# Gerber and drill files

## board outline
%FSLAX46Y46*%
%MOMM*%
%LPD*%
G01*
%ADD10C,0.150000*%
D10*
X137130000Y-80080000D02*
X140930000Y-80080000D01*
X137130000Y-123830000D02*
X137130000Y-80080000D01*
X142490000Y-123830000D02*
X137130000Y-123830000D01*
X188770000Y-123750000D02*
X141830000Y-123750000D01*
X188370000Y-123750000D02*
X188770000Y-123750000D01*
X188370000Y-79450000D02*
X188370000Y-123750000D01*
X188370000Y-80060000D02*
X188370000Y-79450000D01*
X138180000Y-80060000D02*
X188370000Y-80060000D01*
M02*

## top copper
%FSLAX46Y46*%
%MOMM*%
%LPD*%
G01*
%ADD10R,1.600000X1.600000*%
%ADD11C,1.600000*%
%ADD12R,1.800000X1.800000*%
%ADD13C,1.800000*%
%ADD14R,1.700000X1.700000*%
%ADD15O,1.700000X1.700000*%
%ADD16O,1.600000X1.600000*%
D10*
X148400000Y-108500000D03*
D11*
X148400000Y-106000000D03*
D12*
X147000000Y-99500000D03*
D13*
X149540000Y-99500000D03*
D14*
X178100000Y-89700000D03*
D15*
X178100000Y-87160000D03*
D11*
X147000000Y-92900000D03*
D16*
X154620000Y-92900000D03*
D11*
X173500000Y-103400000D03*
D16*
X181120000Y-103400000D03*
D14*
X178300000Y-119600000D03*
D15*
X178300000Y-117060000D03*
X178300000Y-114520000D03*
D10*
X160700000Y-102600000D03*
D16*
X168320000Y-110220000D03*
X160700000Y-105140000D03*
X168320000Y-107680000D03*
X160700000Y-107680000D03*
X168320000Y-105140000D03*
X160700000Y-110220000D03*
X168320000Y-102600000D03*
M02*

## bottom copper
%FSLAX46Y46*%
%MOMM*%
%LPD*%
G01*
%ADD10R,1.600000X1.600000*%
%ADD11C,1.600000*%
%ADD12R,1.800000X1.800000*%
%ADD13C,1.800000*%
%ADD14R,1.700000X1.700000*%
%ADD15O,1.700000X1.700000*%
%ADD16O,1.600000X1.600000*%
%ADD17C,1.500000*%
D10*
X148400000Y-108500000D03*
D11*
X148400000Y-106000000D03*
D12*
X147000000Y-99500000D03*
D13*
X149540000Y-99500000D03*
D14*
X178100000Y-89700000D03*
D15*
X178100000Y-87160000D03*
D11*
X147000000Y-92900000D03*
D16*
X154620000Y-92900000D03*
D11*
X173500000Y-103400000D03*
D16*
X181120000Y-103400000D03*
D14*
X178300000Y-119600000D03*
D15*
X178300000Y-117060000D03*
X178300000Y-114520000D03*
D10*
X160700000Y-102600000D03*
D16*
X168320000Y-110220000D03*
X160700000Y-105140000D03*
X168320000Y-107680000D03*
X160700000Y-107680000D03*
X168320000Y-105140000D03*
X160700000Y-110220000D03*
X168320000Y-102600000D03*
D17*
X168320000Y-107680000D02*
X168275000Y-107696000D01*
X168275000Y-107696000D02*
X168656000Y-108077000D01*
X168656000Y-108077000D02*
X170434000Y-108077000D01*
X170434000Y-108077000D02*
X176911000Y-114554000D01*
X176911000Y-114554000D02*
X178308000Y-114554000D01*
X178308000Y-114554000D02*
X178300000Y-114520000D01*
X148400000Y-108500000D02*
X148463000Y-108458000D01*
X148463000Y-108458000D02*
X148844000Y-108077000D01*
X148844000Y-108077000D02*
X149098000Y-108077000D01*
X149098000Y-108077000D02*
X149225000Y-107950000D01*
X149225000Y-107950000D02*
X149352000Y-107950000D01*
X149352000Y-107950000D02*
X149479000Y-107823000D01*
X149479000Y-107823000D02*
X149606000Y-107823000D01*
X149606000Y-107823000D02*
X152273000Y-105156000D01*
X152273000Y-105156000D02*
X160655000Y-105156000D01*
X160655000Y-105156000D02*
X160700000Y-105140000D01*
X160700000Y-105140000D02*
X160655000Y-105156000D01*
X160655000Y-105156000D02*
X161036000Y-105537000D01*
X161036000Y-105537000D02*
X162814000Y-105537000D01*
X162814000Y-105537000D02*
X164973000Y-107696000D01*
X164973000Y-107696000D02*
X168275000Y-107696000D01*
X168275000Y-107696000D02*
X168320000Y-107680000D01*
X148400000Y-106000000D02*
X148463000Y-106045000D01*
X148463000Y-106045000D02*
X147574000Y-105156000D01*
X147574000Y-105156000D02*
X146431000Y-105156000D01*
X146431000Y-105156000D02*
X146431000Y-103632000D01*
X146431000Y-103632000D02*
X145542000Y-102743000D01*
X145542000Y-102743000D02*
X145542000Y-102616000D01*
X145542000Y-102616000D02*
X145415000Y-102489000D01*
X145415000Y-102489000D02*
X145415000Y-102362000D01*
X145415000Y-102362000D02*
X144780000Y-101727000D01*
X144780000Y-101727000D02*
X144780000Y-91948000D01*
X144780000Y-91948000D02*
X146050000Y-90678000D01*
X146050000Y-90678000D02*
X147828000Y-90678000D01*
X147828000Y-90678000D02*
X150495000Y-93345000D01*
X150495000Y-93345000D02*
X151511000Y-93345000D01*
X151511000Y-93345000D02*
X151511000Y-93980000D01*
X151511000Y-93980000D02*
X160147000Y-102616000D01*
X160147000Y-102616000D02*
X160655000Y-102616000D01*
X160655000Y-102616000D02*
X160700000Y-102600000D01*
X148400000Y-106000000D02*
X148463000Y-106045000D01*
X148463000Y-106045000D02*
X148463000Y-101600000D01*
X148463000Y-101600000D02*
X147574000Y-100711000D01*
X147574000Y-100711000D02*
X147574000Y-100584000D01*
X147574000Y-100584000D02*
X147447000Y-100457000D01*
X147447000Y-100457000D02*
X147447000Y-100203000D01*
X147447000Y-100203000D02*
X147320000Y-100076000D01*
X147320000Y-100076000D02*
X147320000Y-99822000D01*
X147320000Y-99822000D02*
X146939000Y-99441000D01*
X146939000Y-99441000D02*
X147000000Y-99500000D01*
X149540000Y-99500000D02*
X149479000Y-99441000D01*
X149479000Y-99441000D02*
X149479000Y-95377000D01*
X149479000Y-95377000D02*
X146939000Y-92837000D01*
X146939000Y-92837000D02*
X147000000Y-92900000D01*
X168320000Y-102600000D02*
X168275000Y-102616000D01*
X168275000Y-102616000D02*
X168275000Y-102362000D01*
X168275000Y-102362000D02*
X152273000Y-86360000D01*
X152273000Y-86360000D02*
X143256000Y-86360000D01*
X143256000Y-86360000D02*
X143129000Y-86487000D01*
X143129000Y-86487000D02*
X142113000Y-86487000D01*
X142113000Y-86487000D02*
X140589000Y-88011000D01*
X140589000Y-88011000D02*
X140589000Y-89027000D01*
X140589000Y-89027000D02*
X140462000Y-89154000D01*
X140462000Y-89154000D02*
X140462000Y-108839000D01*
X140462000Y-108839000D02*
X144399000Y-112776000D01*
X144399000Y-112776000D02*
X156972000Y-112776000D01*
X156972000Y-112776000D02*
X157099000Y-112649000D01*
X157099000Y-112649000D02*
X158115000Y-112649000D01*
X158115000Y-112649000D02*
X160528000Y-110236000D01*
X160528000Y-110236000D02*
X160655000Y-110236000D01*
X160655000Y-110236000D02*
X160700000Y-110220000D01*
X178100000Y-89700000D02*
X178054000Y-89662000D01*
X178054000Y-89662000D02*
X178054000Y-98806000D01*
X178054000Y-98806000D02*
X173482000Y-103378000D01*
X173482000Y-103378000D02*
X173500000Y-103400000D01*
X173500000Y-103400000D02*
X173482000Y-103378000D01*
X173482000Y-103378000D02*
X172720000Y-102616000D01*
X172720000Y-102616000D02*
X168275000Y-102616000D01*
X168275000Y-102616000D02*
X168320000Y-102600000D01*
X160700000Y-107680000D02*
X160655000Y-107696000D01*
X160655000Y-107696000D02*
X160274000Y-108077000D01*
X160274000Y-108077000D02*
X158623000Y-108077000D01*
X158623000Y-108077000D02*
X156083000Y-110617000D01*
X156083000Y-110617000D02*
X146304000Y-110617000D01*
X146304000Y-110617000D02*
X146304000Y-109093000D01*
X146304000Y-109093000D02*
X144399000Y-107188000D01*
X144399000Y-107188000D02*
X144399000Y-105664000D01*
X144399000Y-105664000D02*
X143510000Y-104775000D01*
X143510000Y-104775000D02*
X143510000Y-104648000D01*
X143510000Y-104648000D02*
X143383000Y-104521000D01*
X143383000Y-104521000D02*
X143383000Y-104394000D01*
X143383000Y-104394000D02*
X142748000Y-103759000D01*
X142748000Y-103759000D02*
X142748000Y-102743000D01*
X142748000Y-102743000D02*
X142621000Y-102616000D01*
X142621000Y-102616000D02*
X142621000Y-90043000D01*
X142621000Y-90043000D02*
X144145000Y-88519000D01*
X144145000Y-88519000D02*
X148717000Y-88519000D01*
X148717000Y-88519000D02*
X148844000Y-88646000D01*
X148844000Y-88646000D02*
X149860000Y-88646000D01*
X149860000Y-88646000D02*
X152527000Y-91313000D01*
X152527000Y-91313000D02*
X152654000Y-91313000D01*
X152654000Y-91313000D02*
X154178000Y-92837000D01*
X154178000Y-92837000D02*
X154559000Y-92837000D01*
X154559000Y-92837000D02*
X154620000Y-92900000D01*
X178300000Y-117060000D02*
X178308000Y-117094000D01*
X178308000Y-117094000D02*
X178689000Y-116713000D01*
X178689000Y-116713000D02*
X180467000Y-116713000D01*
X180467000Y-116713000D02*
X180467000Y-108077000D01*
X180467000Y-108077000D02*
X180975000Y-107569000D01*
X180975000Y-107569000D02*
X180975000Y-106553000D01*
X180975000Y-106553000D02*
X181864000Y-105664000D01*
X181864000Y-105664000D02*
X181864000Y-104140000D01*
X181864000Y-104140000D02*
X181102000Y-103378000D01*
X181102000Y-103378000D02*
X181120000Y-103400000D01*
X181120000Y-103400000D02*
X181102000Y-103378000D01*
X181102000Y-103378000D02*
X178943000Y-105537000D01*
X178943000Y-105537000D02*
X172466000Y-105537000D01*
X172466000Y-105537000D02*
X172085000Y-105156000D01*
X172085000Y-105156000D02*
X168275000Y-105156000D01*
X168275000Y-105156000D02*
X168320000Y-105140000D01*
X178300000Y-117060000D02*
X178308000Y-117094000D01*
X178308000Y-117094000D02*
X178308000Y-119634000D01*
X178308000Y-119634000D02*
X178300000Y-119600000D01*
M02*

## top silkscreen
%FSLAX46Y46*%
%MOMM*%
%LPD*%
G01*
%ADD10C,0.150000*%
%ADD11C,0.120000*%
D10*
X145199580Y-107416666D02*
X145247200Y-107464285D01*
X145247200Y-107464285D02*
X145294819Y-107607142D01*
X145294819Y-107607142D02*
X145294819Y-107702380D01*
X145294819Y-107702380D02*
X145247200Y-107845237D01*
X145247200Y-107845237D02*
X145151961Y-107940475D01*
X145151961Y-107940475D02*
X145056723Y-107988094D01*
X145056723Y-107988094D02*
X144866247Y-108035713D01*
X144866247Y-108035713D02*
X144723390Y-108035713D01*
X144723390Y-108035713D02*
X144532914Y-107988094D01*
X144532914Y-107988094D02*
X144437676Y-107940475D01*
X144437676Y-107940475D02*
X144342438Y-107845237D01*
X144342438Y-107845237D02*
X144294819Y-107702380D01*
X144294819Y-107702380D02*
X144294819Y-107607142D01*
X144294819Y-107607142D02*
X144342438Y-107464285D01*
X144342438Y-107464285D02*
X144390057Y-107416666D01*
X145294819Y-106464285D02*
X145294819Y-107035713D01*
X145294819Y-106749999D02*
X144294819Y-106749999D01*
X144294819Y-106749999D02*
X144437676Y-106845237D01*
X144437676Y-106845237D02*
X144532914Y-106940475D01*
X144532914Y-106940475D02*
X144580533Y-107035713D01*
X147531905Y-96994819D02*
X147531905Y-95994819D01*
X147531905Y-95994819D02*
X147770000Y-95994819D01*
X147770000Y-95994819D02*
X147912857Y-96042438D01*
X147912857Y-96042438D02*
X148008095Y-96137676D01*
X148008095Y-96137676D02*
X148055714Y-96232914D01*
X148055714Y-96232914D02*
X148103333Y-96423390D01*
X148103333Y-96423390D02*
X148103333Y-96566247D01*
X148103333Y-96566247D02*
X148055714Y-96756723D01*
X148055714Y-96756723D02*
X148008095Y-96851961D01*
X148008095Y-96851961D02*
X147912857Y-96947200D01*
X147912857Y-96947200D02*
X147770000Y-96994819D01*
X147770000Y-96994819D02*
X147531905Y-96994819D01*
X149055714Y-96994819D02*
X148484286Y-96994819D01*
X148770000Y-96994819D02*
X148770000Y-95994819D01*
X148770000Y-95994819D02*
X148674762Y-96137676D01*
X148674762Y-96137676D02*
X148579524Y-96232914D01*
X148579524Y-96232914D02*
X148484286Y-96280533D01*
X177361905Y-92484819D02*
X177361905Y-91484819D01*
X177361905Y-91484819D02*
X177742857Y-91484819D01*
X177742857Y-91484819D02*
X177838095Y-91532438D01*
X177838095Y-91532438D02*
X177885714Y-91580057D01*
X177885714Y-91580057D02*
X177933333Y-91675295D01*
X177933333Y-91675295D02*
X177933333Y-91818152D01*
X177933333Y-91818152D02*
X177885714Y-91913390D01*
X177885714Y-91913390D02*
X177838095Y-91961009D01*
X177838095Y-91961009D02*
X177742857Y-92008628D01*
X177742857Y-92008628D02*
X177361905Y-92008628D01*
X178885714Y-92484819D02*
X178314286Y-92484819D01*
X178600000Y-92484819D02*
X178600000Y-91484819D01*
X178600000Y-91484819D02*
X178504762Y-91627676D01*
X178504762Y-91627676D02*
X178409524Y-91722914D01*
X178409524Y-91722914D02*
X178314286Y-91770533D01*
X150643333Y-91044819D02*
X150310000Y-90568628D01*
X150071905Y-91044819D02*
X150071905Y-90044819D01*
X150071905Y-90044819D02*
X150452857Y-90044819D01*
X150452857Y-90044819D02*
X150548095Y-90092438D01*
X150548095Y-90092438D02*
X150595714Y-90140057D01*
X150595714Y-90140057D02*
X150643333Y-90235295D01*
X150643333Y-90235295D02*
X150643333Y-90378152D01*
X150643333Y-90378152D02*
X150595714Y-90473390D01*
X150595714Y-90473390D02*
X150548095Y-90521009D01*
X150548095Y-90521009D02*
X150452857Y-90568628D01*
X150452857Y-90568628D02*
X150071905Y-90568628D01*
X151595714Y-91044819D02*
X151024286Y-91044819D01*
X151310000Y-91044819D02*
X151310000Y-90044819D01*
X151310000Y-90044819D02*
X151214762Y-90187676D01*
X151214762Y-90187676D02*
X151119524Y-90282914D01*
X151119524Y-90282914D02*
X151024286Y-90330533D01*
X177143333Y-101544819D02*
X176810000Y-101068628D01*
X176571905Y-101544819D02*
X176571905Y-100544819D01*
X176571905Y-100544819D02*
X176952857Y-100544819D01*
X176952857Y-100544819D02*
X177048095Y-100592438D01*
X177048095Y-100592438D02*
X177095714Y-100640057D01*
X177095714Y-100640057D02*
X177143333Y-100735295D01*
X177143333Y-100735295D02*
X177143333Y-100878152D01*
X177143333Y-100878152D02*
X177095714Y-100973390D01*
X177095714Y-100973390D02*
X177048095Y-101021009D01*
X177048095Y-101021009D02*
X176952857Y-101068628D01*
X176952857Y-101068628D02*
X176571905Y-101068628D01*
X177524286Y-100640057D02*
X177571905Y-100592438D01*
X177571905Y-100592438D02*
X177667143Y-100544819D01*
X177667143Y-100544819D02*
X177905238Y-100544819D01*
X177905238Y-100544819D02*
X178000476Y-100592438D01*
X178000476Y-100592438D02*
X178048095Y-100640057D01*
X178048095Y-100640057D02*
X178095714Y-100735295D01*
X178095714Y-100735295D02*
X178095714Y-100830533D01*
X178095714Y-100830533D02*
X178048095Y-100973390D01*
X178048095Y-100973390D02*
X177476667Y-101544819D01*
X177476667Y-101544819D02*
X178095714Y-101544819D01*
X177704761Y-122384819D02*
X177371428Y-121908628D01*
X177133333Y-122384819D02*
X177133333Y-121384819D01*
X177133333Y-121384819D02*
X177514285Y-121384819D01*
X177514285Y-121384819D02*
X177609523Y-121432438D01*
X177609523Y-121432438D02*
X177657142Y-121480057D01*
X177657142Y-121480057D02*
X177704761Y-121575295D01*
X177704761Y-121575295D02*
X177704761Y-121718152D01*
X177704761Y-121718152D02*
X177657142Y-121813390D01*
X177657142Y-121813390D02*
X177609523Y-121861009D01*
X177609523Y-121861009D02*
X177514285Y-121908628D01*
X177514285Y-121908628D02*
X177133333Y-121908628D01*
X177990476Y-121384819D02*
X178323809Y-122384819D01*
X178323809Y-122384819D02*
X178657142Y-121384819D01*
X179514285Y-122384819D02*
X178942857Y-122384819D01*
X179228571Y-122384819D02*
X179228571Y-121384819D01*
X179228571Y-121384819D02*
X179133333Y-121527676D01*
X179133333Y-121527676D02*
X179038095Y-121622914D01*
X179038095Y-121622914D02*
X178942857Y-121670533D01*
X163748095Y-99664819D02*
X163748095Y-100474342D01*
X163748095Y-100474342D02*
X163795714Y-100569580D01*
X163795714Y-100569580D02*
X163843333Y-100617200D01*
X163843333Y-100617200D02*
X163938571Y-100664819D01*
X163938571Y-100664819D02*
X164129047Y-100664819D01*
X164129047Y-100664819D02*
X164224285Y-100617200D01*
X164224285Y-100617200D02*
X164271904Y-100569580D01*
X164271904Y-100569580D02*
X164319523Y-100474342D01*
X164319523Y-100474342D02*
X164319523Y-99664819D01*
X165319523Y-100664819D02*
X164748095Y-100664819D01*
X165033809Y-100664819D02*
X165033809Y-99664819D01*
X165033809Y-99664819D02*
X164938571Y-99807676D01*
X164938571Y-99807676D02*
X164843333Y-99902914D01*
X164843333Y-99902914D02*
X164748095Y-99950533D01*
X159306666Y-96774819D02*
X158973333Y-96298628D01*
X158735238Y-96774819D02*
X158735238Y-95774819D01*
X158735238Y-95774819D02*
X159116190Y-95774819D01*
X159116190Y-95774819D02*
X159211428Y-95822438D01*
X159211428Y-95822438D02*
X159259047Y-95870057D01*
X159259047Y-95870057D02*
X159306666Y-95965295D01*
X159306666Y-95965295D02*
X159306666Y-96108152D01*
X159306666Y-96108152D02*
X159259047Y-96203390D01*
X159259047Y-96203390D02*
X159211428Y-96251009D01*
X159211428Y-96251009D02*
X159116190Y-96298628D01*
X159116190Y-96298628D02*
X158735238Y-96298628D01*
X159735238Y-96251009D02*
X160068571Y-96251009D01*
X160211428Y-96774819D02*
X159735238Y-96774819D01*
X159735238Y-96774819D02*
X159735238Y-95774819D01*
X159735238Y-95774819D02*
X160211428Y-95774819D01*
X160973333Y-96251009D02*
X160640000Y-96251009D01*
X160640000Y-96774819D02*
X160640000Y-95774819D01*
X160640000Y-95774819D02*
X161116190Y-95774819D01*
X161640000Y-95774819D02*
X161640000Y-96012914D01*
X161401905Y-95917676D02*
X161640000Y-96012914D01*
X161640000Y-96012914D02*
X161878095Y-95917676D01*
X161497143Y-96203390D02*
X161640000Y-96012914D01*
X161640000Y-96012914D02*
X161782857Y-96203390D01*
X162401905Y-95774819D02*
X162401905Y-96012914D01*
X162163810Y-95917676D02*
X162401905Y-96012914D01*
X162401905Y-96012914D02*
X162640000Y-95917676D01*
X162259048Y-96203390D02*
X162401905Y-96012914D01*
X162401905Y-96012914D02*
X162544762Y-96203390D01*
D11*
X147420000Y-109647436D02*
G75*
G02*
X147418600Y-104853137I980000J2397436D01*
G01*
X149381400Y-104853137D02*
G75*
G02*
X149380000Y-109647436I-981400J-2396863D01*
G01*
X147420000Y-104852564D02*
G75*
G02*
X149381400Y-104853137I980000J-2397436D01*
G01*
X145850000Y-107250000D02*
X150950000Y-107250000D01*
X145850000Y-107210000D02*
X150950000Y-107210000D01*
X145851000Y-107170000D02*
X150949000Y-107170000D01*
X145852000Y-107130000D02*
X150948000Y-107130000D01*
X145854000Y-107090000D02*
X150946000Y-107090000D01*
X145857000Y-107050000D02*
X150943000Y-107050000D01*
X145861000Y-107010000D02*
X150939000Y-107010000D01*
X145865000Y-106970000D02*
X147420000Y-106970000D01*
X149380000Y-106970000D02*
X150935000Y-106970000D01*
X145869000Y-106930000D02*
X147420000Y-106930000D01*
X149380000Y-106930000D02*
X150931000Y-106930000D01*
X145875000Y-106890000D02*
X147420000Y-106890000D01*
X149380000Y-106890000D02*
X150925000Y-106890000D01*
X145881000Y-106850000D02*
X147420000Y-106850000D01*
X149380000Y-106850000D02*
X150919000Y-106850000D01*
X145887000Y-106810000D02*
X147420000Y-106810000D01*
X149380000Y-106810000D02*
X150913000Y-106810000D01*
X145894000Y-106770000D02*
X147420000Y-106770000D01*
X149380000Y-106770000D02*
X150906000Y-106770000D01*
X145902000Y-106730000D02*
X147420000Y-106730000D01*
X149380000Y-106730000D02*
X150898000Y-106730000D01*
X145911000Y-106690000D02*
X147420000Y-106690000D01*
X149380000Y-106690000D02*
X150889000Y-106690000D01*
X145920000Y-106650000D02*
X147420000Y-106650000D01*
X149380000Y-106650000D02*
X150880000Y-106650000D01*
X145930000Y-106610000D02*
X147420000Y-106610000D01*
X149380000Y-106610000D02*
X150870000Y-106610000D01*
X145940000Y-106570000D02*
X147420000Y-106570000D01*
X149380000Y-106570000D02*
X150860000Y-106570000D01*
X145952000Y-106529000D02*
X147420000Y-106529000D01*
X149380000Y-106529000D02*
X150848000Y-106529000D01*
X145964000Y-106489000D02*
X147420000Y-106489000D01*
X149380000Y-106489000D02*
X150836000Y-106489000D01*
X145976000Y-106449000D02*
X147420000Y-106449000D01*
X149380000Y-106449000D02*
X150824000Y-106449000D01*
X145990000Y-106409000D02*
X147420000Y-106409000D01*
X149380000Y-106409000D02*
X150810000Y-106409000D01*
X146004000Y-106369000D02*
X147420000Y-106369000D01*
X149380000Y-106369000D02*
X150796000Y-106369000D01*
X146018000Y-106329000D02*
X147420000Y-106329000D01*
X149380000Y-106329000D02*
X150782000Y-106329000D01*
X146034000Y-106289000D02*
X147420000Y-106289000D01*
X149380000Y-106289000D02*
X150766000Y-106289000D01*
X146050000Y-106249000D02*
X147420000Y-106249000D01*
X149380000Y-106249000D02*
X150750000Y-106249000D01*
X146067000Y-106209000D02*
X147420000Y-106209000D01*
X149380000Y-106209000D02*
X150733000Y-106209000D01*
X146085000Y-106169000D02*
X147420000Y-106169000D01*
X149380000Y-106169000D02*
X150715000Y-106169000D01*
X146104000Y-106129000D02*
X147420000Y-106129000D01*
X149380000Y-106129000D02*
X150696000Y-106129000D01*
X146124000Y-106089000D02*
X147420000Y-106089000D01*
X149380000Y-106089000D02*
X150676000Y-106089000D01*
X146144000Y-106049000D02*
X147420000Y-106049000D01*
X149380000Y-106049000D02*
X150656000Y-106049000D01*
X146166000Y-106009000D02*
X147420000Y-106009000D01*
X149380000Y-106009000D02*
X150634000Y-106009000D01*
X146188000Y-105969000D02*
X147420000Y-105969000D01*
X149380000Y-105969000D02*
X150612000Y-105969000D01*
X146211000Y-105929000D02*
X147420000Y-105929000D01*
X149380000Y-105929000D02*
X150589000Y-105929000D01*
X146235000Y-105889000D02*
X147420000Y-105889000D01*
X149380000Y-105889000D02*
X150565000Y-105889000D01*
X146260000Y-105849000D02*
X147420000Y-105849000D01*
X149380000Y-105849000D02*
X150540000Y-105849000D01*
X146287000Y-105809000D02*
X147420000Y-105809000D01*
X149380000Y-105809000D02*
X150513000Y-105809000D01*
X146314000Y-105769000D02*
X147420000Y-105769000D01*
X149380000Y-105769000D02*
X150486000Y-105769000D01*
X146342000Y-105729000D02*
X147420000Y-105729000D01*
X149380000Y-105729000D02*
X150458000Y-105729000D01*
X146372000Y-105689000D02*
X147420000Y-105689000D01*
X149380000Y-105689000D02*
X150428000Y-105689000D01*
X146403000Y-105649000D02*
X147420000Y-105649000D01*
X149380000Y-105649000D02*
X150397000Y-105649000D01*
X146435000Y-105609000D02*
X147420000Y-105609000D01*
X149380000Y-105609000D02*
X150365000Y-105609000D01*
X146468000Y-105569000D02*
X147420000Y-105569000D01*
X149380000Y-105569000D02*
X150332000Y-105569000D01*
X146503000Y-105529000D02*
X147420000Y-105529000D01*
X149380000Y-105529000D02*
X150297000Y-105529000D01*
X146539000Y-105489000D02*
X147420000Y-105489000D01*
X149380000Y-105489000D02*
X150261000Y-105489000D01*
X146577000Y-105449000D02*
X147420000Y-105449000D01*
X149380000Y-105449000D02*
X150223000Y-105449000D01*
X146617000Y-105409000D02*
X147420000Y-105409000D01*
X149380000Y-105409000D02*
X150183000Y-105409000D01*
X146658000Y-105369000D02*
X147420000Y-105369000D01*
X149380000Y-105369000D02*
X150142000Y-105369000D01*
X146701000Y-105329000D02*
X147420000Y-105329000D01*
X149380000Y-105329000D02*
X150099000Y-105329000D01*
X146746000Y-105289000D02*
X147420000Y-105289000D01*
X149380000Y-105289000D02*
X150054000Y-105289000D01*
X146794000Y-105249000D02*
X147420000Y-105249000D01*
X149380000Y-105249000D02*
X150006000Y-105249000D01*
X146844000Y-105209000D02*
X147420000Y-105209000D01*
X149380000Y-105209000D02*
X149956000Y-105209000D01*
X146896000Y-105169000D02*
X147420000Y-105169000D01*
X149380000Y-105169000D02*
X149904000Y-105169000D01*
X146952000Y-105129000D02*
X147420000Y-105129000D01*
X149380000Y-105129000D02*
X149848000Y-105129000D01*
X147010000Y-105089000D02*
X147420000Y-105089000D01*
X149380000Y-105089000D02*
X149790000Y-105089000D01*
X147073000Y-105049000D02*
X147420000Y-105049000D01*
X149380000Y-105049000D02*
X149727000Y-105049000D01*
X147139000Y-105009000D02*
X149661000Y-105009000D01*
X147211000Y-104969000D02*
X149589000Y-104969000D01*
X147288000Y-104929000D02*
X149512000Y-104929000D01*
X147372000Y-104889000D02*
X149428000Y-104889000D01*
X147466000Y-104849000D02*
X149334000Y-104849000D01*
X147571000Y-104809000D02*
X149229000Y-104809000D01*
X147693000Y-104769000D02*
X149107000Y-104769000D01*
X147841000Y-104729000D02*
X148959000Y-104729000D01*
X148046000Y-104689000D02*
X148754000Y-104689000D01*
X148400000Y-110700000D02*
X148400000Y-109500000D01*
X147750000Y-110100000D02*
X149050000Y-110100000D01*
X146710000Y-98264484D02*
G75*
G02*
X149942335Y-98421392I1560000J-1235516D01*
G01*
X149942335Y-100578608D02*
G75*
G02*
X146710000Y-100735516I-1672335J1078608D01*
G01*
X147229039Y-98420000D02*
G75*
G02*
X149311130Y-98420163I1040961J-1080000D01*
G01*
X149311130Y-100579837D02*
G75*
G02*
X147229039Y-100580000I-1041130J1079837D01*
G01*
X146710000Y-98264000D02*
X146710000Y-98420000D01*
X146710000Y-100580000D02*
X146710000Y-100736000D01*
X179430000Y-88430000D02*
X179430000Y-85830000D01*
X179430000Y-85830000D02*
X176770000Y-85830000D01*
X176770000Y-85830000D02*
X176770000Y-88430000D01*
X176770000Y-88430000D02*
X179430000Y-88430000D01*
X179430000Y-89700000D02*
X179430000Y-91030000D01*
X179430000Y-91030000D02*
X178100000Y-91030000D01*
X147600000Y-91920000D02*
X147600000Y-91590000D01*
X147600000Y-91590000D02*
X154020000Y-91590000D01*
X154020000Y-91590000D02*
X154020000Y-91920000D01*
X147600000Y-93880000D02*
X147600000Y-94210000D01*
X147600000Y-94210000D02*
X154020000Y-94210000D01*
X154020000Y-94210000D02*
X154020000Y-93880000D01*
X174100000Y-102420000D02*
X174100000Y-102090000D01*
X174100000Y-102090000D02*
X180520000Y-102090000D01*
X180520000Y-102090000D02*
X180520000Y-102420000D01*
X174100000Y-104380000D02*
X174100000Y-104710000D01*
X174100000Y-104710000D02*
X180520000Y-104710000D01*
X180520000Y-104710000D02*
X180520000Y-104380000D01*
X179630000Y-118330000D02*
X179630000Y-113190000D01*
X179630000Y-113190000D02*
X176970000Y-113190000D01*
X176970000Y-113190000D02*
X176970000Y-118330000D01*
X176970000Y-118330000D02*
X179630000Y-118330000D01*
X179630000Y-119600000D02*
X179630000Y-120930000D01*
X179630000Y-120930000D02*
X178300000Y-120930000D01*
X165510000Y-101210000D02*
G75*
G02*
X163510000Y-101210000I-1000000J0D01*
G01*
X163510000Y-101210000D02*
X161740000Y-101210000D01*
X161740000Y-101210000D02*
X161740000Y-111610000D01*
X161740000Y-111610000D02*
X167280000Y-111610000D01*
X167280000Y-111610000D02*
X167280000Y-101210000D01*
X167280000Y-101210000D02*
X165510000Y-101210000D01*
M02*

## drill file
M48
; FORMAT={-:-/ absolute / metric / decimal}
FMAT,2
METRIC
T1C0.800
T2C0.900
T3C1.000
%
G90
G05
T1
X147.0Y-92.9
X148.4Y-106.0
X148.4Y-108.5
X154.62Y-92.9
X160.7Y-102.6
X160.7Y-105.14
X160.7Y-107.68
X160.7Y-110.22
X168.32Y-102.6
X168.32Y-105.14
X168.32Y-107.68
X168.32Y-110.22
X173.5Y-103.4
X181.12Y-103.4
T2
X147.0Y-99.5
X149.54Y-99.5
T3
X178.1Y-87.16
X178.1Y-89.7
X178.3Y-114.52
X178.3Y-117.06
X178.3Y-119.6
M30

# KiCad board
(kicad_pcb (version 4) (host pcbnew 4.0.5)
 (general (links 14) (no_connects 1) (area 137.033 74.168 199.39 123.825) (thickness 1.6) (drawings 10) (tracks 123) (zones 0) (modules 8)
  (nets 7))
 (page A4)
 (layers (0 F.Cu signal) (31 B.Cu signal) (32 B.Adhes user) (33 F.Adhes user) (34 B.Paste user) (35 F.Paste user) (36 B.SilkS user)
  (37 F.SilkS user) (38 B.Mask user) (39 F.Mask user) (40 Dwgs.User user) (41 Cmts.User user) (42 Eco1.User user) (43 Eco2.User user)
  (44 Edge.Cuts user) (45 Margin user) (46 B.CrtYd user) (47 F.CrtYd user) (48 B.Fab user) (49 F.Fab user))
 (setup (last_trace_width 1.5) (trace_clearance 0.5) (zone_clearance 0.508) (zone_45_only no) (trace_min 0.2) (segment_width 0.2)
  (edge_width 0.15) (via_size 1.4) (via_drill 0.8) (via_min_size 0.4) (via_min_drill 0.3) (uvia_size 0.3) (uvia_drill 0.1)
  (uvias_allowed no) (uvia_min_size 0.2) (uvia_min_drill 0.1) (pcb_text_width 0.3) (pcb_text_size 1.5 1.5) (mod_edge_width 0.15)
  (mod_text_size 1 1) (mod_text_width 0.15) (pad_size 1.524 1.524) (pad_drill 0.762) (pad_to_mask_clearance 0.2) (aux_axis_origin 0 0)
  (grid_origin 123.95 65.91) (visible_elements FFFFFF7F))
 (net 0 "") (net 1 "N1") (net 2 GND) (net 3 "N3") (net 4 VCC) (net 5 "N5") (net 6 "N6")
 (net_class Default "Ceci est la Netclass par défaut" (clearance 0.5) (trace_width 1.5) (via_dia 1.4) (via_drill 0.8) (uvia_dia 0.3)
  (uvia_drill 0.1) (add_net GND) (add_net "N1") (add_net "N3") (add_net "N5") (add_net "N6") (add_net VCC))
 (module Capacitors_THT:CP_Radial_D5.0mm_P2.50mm (layer F.Cu) (at 148.4 108.5 90)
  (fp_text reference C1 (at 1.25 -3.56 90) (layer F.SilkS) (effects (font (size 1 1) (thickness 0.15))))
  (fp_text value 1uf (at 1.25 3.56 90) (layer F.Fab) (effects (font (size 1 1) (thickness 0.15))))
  (fp_arc (start 1.25 0) (end -1.147436 -0.98) (angle 135.5) (layer F.SilkS) (width 0.12))
  (fp_arc (start 1.25 0) (end -1.147436 0.98) (angle -135.5) (layer F.SilkS) (width 0.12))
  (fp_arc (start 1.25 0) (end 3.647436 -0.98) (angle 44.5) (layer F.SilkS) (width 0.12))
  (fp_line (start 1.25 -2.55) (end 1.25 2.55) (layer F.SilkS) (width 0.12))
  (fp_line (start 1.29 -2.55) (end 1.29 2.55) (layer F.SilkS) (width 0.12))
  (fp_line (start 1.33 -2.549) (end 1.33 2.549) (layer F.SilkS) (width 0.12))
  (fp_line (start 1.37 -2.548) (end 1.37 2.548) (layer F.SilkS) (width 0.12))
  (fp_line (start 1.41 -2.546) (end 1.41 2.546) (layer F.SilkS) (width 0.12))
  (fp_line (start 1.45 -2.543) (end 1.45 2.543) (layer F.SilkS) (width 0.12))
  (fp_line (start 1.49 -2.539) (end 1.49 2.539) (layer F.SilkS) (width 0.12))
  (fp_line (start 1.53 -2.535) (end 1.53 -0.98) (layer F.SilkS) (width 0.12))
  (fp_line (start 1.53 0.98) (end 1.53 2.535) (layer F.SilkS) (width 0.12))
  (fp_line (start 1.57 -2.531) (end 1.57 -0.98) (layer F.SilkS) (width 0.12))
  (fp_line (start 1.57 0.98) (end 1.57 2.531) (layer F.SilkS) (width 0.12))
  (fp_line (start 1.61 -2.525) (end 1.61 -0.98) (layer F.SilkS) (width 0.12))
  (fp_line (start 1.61 0.98) (end 1.61 2.525) (layer F.SilkS) (width 0.12))
  (fp_line (start 1.65 -2.519) (end 1.65 -0.98) (layer F.SilkS) (width 0.12))
  (fp_line (start 1.65 0.98) (end 1.65 2.519) (layer F.SilkS) (width 0.12))
  (fp_line (start 1.69 -2.513) (end 1.69 -0.98) (layer F.SilkS) (width 0.12))
  (fp_line (start 1.69 0.98) (end 1.69 2.513) (layer F.SilkS) (width 0.12))
  (fp_line (start 1.73 -2.506) (end 1.73 -0.98) (layer F.SilkS) (width 0.12))
  (fp_line (start 1.73 0.98) (end 1.73 2.506) (layer F.SilkS) (width 0.12))
  (fp_line (start 1.77 -2.498) (end 1.77 -0.98) (layer F.SilkS) (width 0.12))
  (fp_line (start 1.77 0.98) (end 1.77 2.498) (layer F.SilkS) (width 0.12))
  (fp_line (start 1.81 -2.489) (end 1.81 -0.98) (layer F.SilkS) (width 0.12))
  (fp_line (start 1.81 0.98) (end 1.81 2.489) (layer F.SilkS) (width 0.12))
  (fp_line (start 1.85 -2.48) (end 1.85 -0.98) (layer F.SilkS) (width 0.12))
  (fp_line (start 1.85 0.98) (end 1.85 2.48) (layer F.SilkS) (width 0.12))
  (fp_line (start 1.89 -2.47) (end 1.89 -0.98) (layer F.SilkS) (width 0.12))
  (fp_line (start 1.89 0.98) (end 1.89 2.47) (layer F.SilkS) (width 0.12))
  (fp_line (start 1.93 -2.46) (end 1.93 -0.98) (layer F.SilkS) (width 0.12))
  (fp_line (start 1.93 0.98) (end 1.93 2.46) (layer F.SilkS) (width 0.12))
  (fp_line (start 1.971 -2.448) (end 1.971 -0.98) (layer F.SilkS) (width 0.12))
  (fp_line (start 1.971 0.98) (end 1.971 2.448) (layer F.SilkS) (width 0.12))
  (fp_line (start 2.011 -2.436) (end 2.011 -0.98) (layer F.SilkS) (width 0.12))
  (fp_line (start 2.011 0.98) (end 2.011 2.436) (layer F.SilkS) (width 0.12))
  (fp_line (start 2.051 -2.424) (end 2.051 -0.98) (layer F.SilkS) (width 0.12))
  (fp_line (start 2.051 0.98) (end 2.051 2.424) (layer F.SilkS) (width 0.12))
  (fp_line (start 2.091 -2.41) (end 2.091 -0.98) (layer F.SilkS) (width 0.12))
  (fp_line (start 2.091 0.98) (end 2.091 2.41) (layer F.SilkS) (width 0.12))
  (fp_line (start 2.131 -2.396) (end 2.131 -0.98) (layer F.SilkS) (width 0.12))
  (fp_line (start 2.131 0.98) (end 2.131 2.396) (layer F.SilkS) (width 0.12))
  (fp_line (start 2.171 -2.382) (end 2.171 -0.98) (layer F.SilkS) (width 0.12))
  (fp_line (start 2.171 0.98) (end 2.171 2.382) (layer F.SilkS) (width 0.12))
  (fp_line (start 2.211 -2.366) (end 2.211 -0.98) (layer F.SilkS) (width 0.12))
  (fp_line (start 2.211 0.98) (end 2.211 2.366) (layer F.SilkS) (width 0.12))
  (fp_line (start 2.251 -2.35) (end 2.251 -0.98) (layer F.SilkS) (width 0.12))
  (fp_line (start 2.251 0.98) (end 2.251 2.35) (layer F.SilkS) (width 0.12))
  (fp_line (start 2.291 -2.333) (end 2.291 -0.98) (layer F.SilkS) (width 0.12))
  (fp_line (start 2.291 0.98) (end 2.291 2.333) (layer F.SilkS) (width 0.12))
  (fp_line (start 2.331 -2.315) (end 2.331 -0.98) (layer F.SilkS) (width 0.12))
  (fp_line (start 2.331 0.98) (end 2.331 2.315) (layer F.SilkS) (width 0.12))
  (fp_line (start 2.371 -2.296) (end 2.371 -0.98) (layer F.SilkS) (width 0.12))
  (fp_line (start 2.371 0.98) (end 2.371 2.296) (layer F.SilkS) (width 0.12))
  (fp_line (start 2.411 -2.276) (end 2.411 -0.98) (layer F.SilkS) (width 0.12))
  (fp_line (start 2.411 0.98) (end 2.411 2.276) (layer F.SilkS) (width 0.12))
  (fp_line (start 2.451 -2.256) (end 2.451 -0.98) (layer F.SilkS) (width 0.12))
  (fp_line (start 2.451 0.98) (end 2.451 2.256) (layer F.SilkS) (width 0.12))
  (fp_line (start 2.491 -2.234) (end 2.491 -0.98) (layer F.SilkS) (width 0.12))
  (fp_line (start 2.491 0.98) (end 2.491 2.234) (layer F.SilkS) (width 0.12))
  (fp_line (start 2.531 -2.212) (end 2.531 -0.98) (layer F.SilkS) (width 0.12))
  (fp_line (start 2.531 0.98) (end 2.531 2.212) (layer F.SilkS) (width 0.12))
  (fp_line (start 2.571 -2.189) (end 2.571 -0.98) (layer F.SilkS) (width 0.12))
  (fp_line (start 2.571 0.98) (end 2.571 2.189) (layer F.SilkS) (width 0.12))
  (fp_line (start 2.611 -2.165) (end 2.611 -0.98) (layer F.SilkS) (width 0.12))
  (fp_line (start 2.611 0.98) (end 2.611 2.165) (layer F.SilkS) (width 0.12))
  (fp_line (start 2.651 -2.14) (end 2.651 -0.98) (layer F.SilkS) (width 0.12))
  (fp_line (start 2.651 0.98) (end 2.651 2.14) (layer F.SilkS) (width 0.12))
  (fp_line (start 2.691 -2.113) (end 2.691 -0.98) (layer F.SilkS) (width 0.12))
  (fp_line (start 2.691 0.98) (end 2.691 2.113) (layer F.SilkS) (width 0.12))
  (fp_line (start 2.731 -2.086) (end 2.731 -0.98) (layer F.SilkS) (width 0.12))
  (fp_line (start 2.731 0.98) (end 2.731 2.086) (layer F.SilkS) (width 0.12))
  (fp_line (start 2.771 -2.058) (end 2.771 -0.98) (layer F.SilkS) (width 0.12))
  (fp_line (start 2.771 0.98) (end 2.771 2.058) (layer F.SilkS) (width 0.12))
  (fp_line (start 2.811 -2.028) (end 2.811 -0.98) (layer F.SilkS) (width 0.12))
  (fp_line (start 2.811 0.98) (end 2.811 2.028) (layer F.SilkS) (width 0.12))
  (fp_line (start 2.851 -1.997) (end 2.851 -0.98) (layer F.SilkS) (width 0.12))
  (fp_line (start 2.851 0.98) (end 2.851 1.997) (layer F.SilkS) (width 0.12))
  (fp_line (start 2.891 -1.965) (end 2.891 -0.98) (layer F.SilkS) (width 0.12))
  (fp_line (start 2.891 0.98) (end 2.891 1.965) (layer F.SilkS) (width 0.12))
  (fp_line (start 2.931 -1.932) (end 2.931 -0.98) (layer F.SilkS) (width 0.12))
  (fp_line (start 2.931 0.98) (end 2.931 1.932) (layer F.SilkS) (width 0.12))
  (fp_line (start 2.971 -1.897) (end 2.971 -0.98) (layer F.SilkS) (width 0.12))
  (fp_line (start 2.971 0.98) (end 2.971 1.897) (layer F.SilkS) (width 0.12))
  (fp_line (start 3.011 -1.861) (end 3.011 -0.98) (layer F.SilkS) (width 0.12))
  (fp_line (start 3.011 0.98) (end 3.011 1.861) (layer F.SilkS) (width 0.12))
  (fp_line (start 3.051 -1.823) (end 3.051 -0.98) (layer F.SilkS) (width 0.12))
  (fp_line (start 3.051 0.98) (end 3.051 1.823) (layer F.SilkS) (width 0.12))
  (fp_line (start 3.091 -1.783) (end 3.091 -0.98) (layer F.SilkS) (width 0.12))
  (fp_line (start 3.091 0.98) (end 3.091 1.783) (layer F.SilkS) (width 0.12))
  (fp_line (start 3.131 -1.742) (end 3.131 -0.98) (layer F.SilkS) (width 0.12))
  (fp_line (start 3.131 0.98) (end 3.131 1.742) (layer F.SilkS) (width 0.12))
  (fp_line (start 3.171 -1.699) (end 3.171 -0.98) (layer F.SilkS) (width 0.12))
  (fp_line (start 3.171 0.98) (end 3.171 1.699) (layer F.SilkS) (width 0.12))
  (fp_line (start 3.211 -1.654) (end 3.211 -0.98) (layer F.SilkS) (width 0.12))
  (fp_line (start 3.211 0.98) (end 3.211 1.654) (layer F.SilkS) (width 0.12))
  (fp_line (start 3.251 -1.606) (end 3.251 -0.98) (layer F.SilkS) (width 0.12))
  (fp_line (start 3.251 0.98) (end 3.251 1.606) (layer F.SilkS) (width 0.12))
  (fp_line (start 3.291 -1.556) (end 3.291 -0.98) (layer F.SilkS) (width 0.12))
  (fp_line (start 3.291 0.98) (end 3.291 1.556) (layer F.SilkS) (width 0.12))
  (fp_line (start 3.331 -1.504) (end 3.331 -0.98) (layer F.SilkS) (width 0.12))
  (fp_line (start 3.331 0.98) (end 3.331 1.504) (layer F.SilkS) (width 0.12))
  (fp_line (start 3.371 -1.448) (end 3.371 -0.98) (layer F.SilkS) (width 0.12))
  (fp_line (start 3.371 0.98) (end 3.371 1.448) (layer F.SilkS) (width 0.12))
  (fp_line (start 3.411 -1.39) (end 3.411 -0.98) (layer F.SilkS) (width 0.12))
  (fp_line (start 3.411 0.98) (end 3.411 1.39) (layer F.SilkS) (width 0.12))
  (fp_line (start 3.451 -1.327) (end 3.451 -0.98) (layer F.SilkS) (width 0.12))
  (fp_line (start 3.451 0.98) (end 3.451 1.327) (layer F.SilkS) (width 0.12))
  (fp_line (start 3.491 -1.261) (end 3.491 1.261) (layer F.SilkS) (width 0.12))
  (fp_line (start 3.531 -1.189) (end 3.531 1.189) (layer F.SilkS) (width 0.12))
  (fp_line (start 3.571 -1.112) (end 3.571 1.112) (layer F.SilkS) (width 0.12))
  (fp_line (start 3.611 -1.028) (end 3.611 1.028) (layer F.SilkS) (width 0.12))
  (fp_line (start 3.651 -0.934) (end 3.651 0.934) (layer F.SilkS) (width 0.12))
  (fp_line (start 3.691 -0.829) (end 3.691 0.829) (layer F.SilkS) (width 0.12))
  (fp_line (start 3.731 -0.707) (end 3.731 0.707) (layer F.SilkS) (width 0.12))
  (fp_line (start 3.771 -0.559) (end 3.771 0.559) (layer F.SilkS) (width 0.12))
  (fp_line (start 3.811 -0.354) (end 3.811 0.354) (layer F.SilkS) (width 0.12))
  (fp_line (start -2.2 0) (end -1 0) (layer F.SilkS) (width 0.12))
  (fp_line (start -1.6 -0.65) (end -1.6 0.65) (layer F.SilkS) (width 0.12))
  (pad 1 thru_hole rect (at 0 0 90) (size 1.6 1.6) (drill 0.8) (layers *.Cu *.Mask) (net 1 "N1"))
  (pad 2 thru_hole circle (at 2.5 0 90) (size 1.6 1.6) (drill 0.8) (layers *.Cu *.Mask) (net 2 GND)))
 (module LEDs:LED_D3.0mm (layer F.Cu) (at 147 99.5)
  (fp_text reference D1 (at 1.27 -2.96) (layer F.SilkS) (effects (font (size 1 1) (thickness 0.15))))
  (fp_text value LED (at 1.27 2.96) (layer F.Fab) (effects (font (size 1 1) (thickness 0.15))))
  (fp_arc (start 1.27 0) (end -0.29 -1.235516) (angle 108.8) (layer F.SilkS) (width 0.12))
  (fp_arc (start 1.27 0) (end -0.29 1.235516) (angle -108.8) (layer F.SilkS) (width 0.12))
  (fp_arc (start 1.27 0) (end 0.229039 -1.08) (angle 87.9) (layer F.SilkS) (width 0.12))
  (fp_arc (start 1.27 0) (end 0.229039 1.08) (angle -87.9) (layer F.SilkS) (width 0.12))
  (fp_line (start -0.29 -1.236) (end -0.29 -1.08) (layer F.SilkS) (width 0.12))
  (fp_line (start -0.29 1.08) (end -0.29 1.236) (layer F.SilkS) (width 0.12))
  (pad 1 thru_hole rect (at 0 0) (size 1.8 1.8) (drill 0.9) (layers *.Cu *.Mask) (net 2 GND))
  (pad 2 thru_hole circle (at 2.54 0) (size 1.8 1.8) (drill 0.9) (layers *.Cu *.Mask) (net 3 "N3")))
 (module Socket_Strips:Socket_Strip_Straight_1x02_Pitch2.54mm (layer F.Cu) (at 178.1 89.7 180)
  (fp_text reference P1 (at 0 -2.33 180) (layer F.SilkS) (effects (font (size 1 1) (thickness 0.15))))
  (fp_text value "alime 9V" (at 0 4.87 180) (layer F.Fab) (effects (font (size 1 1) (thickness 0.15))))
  (fp_line (start -1.33 1.27) (end -1.33 3.87) (layer F.SilkS) (width 0.12))
  (fp_line (start -1.33 3.87) (end 1.33 3.87) (layer F.SilkS) (width 0.12))
  (fp_line (start 1.33 3.87) (end 1.33 1.27) (layer F.SilkS) (width 0.12))
  (fp_line (start 1.33 1.27) (end -1.33 1.27) (layer F.SilkS) (width 0.12))
  (fp_line (start -1.33 0) (end -1.33 -1.33) (layer F.SilkS) (width 0.12))
  (fp_line (start -1.33 -1.33) (end 0 -1.33) (layer F.SilkS) (width 0.12))
  (pad 1 thru_hole rect (at 0 0 180) (size 1.7 1.7) (drill 1) (layers *.Cu *.Mask) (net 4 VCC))
  (pad 2 thru_hole oval (at 0 2.54 180) (size 1.7 1.7) (drill 1) (layers *.Cu *.Mask) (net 2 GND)))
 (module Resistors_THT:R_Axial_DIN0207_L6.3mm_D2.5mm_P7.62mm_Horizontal (layer F.Cu) (at 147 92.9)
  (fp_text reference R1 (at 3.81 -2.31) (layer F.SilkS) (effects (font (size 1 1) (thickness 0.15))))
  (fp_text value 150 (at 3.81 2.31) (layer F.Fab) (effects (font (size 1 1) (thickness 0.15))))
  (fp_line (start 0.6 -0.98) (end 0.6 -1.31) (layer F.SilkS) (width 0.12))
  (fp_line (start 0.6 -1.31) (end 7.02 -1.31) (layer F.SilkS) (width 0.12))
  (fp_line (start 7.02 -1.31) (end 7.02 -0.98) (layer F.SilkS) (width 0.12))
  (fp_line (start 0.6 0.98) (end 0.6 1.31) (layer F.SilkS) (width 0.12))
  (fp_line (start 0.6 1.31) (end 7.02 1.31) (layer F.SilkS) (width 0.12))
  (fp_line (start 7.02 1.31) (end 7.02 0.98) (layer F.SilkS) (width 0.12))
  (pad 1 thru_hole circle (at 0 0) (size 1.6 1.6) (drill 0.8) (layers *.Cu *.Mask) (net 3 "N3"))
  (pad 2 thru_hole oval (at 7.62 0) (size 1.6 1.6) (drill 0.8) (layers *.Cu *.Mask) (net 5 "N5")))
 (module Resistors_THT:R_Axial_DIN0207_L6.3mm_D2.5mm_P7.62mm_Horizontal (layer F.Cu) (at 173.5 103.4)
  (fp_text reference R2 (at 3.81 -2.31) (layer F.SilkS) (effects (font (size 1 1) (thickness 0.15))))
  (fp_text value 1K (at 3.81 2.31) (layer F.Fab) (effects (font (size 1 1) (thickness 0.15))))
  (fp_line (start 0.6 -0.98) (end 0.6 -1.31) (layer F.SilkS) (width 0.12))
  (fp_line (start 0.6 -1.31) (end 7.02 -1.31) (layer F.SilkS) (width 0.12))
  (fp_line (start 7.02 -1.31) (end 7.02 -0.98) (layer F.SilkS) (width 0.12))
  (fp_line (start 0.6 0.98) (end 0.6 1.31) (layer F.SilkS) (width 0.12))
  (fp_line (start 0.6 1.31) (end 7.02 1.31) (layer F.SilkS) (width 0.12))
  (fp_line (start 7.02 1.31) (end 7.02 0.98) (layer F.SilkS) (width 0.12))
  (pad 1 thru_hole circle (at 0 0) (size 1.6 1.6) (drill 0.8) (layers *.Cu *.Mask) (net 4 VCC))
  (pad 2 thru_hole oval (at 7.62 0) (size 1.6 1.6) (drill 0.8) (layers *.Cu *.Mask) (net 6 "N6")))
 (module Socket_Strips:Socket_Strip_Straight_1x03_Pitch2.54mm (layer F.Cu) (at 178.3 119.6 180)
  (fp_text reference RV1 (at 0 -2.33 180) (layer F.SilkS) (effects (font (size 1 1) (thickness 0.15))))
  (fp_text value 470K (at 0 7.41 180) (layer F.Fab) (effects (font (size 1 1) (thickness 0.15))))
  (fp_line (start -1.33 1.27) (end -1.33 6.41) (layer F.SilkS) (width 0.12))
  (fp_line (start -1.33 6.41) (end 1.33 6.41) (layer F.SilkS) (width 0.12))
  (fp_line (start 1.33 6.41) (end 1.33 1.27) (layer F.SilkS) (width 0.12))
  (fp_line (start 1.33 1.27) (end -1.33 1.27) (layer F.SilkS) (width 0.12))
  (fp_line (start -1.33 0) (end -1.33 -1.33) (layer F.SilkS) (width 0.12))
  (fp_line (start -1.33 -1.33) (end 0 -1.33) (layer F.SilkS) (width 0.12))
  (pad 1 thru_hole rect (at 0 0 180) (size 1.7 1.7) (drill 1) (layers *.Cu *.Mask) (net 6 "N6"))
  (pad 2 thru_hole oval (at 0 2.54 180) (size 1.7 1.7) (drill 1) (layers *.Cu *.Mask) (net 6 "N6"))
  (pad 3 thru_hole oval (at 0 5.08 180) (size 1.7 1.7) (drill 1) (layers *.Cu *.Mask) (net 1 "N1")))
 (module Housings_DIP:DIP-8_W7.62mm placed (layer F.Cu) (at 160.7 102.6)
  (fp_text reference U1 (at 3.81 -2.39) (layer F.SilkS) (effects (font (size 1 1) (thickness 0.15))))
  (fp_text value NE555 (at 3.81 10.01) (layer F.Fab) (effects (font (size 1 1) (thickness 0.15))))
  (fp_arc (start 3.81 -1.39) (end 2.81 -1.39) (angle -180) (layer F.SilkS) (width 0.12))
  (fp_line (start 2.81 -1.39) (end 1.04 -1.39) (layer F.SilkS) (width 0.12))
  (fp_line (start 1.04 -1.39) (end 1.04 9.01) (layer F.SilkS) (width 0.12))
  (fp_line (start 1.04 9.01) (end 6.58 9.01) (layer F.SilkS) (width 0.12))
  (fp_line (start 6.58 9.01) (end 6.58 -1.39) (layer F.SilkS) (width 0.12))
  (fp_line (start 6.58 -1.39) (end 4.81 -1.39) (layer F.SilkS) (width 0.12))
  (pad 1 thru_hole rect (at 0 0) (size 1.6 1.6) (drill 0.8) (layers *.Cu *.Mask) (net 2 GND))
  (pad 5 thru_hole oval (at 7.62 7.62) (size 1.6 1.6) (drill 0.8) (layers *.Cu *.Mask))
  (pad 2 thru_hole oval (at 0 2.54) (size 1.6 1.6) (drill 0.8) (layers *.Cu *.Mask) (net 1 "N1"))
  (pad 6 thru_hole oval (at 7.62 5.08) (size 1.6 1.6) (drill 0.8) (layers *.Cu *.Mask) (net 1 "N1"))
  (pad 3 thru_hole oval (at 0 5.08) (size 1.6 1.6) (drill 0.8) (layers *.Cu *.Mask) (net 5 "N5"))
  (pad 7 thru_hole oval (at 7.62 2.54) (size 1.6 1.6) (drill 0.8) (layers *.Cu *.Mask) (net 6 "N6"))
  (pad 4 thru_hole oval (at 0 7.62) (size 1.6 1.6) (drill 0.8) (layers *.Cu *.Mask) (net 4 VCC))
  (pad 8 thru_hole oval (at 7.62 0) (size 1.6 1.6) (drill 0.8) (layers *.Cu *.Mask) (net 4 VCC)))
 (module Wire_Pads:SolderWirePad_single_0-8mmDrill (layer F.Cu) (at 160.64 98.86)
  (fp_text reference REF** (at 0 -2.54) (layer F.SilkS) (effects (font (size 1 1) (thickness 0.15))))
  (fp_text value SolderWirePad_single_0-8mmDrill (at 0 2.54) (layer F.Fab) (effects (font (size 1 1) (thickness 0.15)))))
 (gr_line (start 137.13 80.08) (end 140.93 80.08) (angle 90) (layer Edge.Cuts) (width 0.15))
 (gr_line (start 137.13 123.83) (end 137.13 80.08) (angle 90) (layer Edge.Cuts) (width 0.15))
 (gr_line (start 142.49 123.83) (end 137.13 123.83) (angle 90) (layer Edge.Cuts) (width 0.15))
 (gr_line (start 188.77 123.75) (end 141.83 123.75) (angle 90) (layer Edge.Cuts) (width 0.15))
 (gr_line (start 188.37 123.75) (end 188.77 123.75) (angle 90) (layer Edge.Cuts) (width 0.15))
 (gr_line (start 188.37 79.45) (end 188.37 123.75) (angle 90) (layer Edge.Cuts) (width 0.15))
 (gr_line (start 188.37 80.06) (end 188.37 79.45) (angle 90) (layer Edge.Cuts) (width 0.15))
 (gr_line (start 138.18 80.06) (end 188.37 80.06) (angle 90) (layer Edge.Cuts) (width 0.15))
 (segment (start 168.32 107.68) (end 168.275 107.696) (width 1.5) (layer B.Cu) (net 1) (status 80000))
 (segment (start 168.275 107.696) (end 168.656 108.077) (width 1.5) (layer B.Cu) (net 1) (status 80000))
 (segment (start 168.656 108.077) (end 170.434 108.077) (width 1.5) (layer B.Cu) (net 1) (status 80000))
 (segment (start 170.434 108.077) (end 176.911 114.554) (width 1.5) (layer B.Cu) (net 1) (status 80000))
 (segment (start 176.911 114.554) (end 178.308 114.554) (width 1.5) (layer B.Cu) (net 1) (status 80000))
 (segment (start 178.308 114.554) (end 178.3 114.52) (width 1.5) (layer B.Cu) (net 1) (status 80000))
 (segment (start 148.4 108.5) (end 148.463 108.458) (width 1.5) (layer B.Cu) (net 1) (status 80000))
 (segment (start 148.463 108.458) (end 148.844 108.077) (width 1.5) (layer B.Cu) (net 1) (status 80000))
 (segment (start 148.844 108.077) (end 149.098 108.077) (width 1.5) (layer B.Cu) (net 1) (status 80000))
 (segment (start 149.098 108.077) (end 149.225 107.95) (width 1.5) (layer B.Cu) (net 1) (status 80000))
 (segment (start 149.225 107.95) (end 149.352 107.95) (width 1.5) (layer B.Cu) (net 1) (status 80000))
 (segment (start 149.352 107.95) (end 149.479 107.823) (width 1.5) (layer B.Cu) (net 1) (status 80000))
 (segment (start 149.479 107.823) (end 149.606 107.823) (width 1.5) (layer B.Cu) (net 1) (status 80000))
 (segment (start 149.606 107.823) (end 152.273 105.156) (width 1.5) (layer B.Cu) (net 1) (status 80000))
 (segment (start 152.273 105.156) (end 160.655 105.156) (width 1.5) (layer B.Cu) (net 1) (status 80000))
 (segment (start 160.655 105.156) (end 160.7 105.14) (width 1.5) (layer B.Cu) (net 1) (status 80000))
 (segment (start 160.7 105.14) (end 160.655 105.156) (width 1.5) (layer B.Cu) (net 1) (status 80000))
 (segment (start 160.655 105.156) (end 161.036 105.537) (width 1.5) (layer B.Cu) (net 1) (status 80000))
 (segment (start 161.036 105.537) (end 162.814 105.537) (width 1.5) (layer B.Cu) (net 1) (status 80000))
 (segment (start 162.814 105.537) (end 164.973 107.696) (width 1.5) (layer B.Cu) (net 1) (status 80000))
 (segment (start 164.973 107.696) (end 168.275 107.696) (width 1.5) (layer B.Cu) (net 1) (status 80000))
 (segment (start 168.275 107.696) (end 168.32 107.68) (width 1.5) (layer B.Cu) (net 1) (status 80000))
 (segment (start 148.4 106) (end 148.463 106.045) (width 1.5) (layer B.Cu) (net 2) (status 80000))
 (segment (start 148.463 106.045) (end 147.574 105.156) (width 1.5) (layer B.Cu) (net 2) (status 80000))
 (segment (start 147.574 105.156) (end 146.431 105.156) (width 1.5) (layer B.Cu) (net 2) (status 80000))
 (segment (start 146.431 105.156) (end 146.431 103.632) (width 1.5) (layer B.Cu) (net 2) (status 80000))
 (segment (start 146.431 103.632) (end 145.542 102.743) (width 1.5) (layer B.Cu) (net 2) (status 80000))
 (segment (start 145.542 102.743) (end 145.542 102.616) (width 1.5) (layer B.Cu) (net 2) (status 80000))
 (segment (start 145.542 102.616) (end 145.415 102.489) (width 1.5) (layer B.Cu) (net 2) (status 80000))
 (segment (start 145.415 102.489) (end 145.415 102.362) (width 1.5) (layer B.Cu) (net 2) (status 80000))
 (segment (start 145.415 102.362) (end 144.78 101.727) (width 1.5) (layer B.Cu) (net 2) (status 80000))
 (segment (start 144.78 101.727) (end 144.78 91.948) (width 1.5) (layer B.Cu) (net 2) (status 80000))
 (segment (start 144.78 91.948) (end 146.05 90.678) (width 1.5) (layer B.Cu) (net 2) (status 80000))
 (segment (start 146.05 90.678) (end 147.828 90.678) (width 1.5) (layer B.Cu) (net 2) (status 80000))
 (segment (start 147.828 90.678) (end 150.495 93.345) (width 1.5) (layer B.Cu) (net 2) (status 80000))
 (segment (start 150.495 93.345) (end 151.511 93.345) (width 1.5) (layer B.Cu) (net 2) (status 80000))
 (segment (start 151.511 93.345) (end 151.511 93.98) (width 1.5) (layer B.Cu) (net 2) (status 80000))
 (segment (start 151.511 93.98) (end 160.147 102.616) (width 1.5) (layer B.Cu) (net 2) (status 80000))
 (segment (start 160.147 102.616) (end 160.655 102.616) (width 1.5) (layer B.Cu) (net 2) (status 80000))
 (segment (start 160.655 102.616) (end 160.7 102.6) (width 1.5) (layer B.Cu) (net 2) (status 80000))
 (segment (start 148.4 106) (end 148.463 106.045) (width 1.5) (layer B.Cu) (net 2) (status 80000))
 (segment (start 148.463 106.045) (end 148.463 101.6) (width 1.5) (layer B.Cu) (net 2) (status 80000))
 (segment (start 148.463 101.6) (end 147.574 100.711) (width 1.5) (layer B.Cu) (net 2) (status 80000))
 (segment (start 147.574 100.711) (end 147.574 100.584) (width 1.5) (layer B.Cu) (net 2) (status 80000))
 (segment (start 147.574 100.584) (end 147.447 100.457) (width 1.5) (layer B.Cu) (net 2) (status 80000))
 (segment (start 147.447 100.457) (end 147.447 100.203) (width 1.5) (layer B.Cu) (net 2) (status 80000))
 (segment (start 147.447 100.203) (end 147.32 100.076) (width 1.5) (layer B.Cu) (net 2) (status 80000))
 (segment (start 147.32 100.076) (end 147.32 99.822) (width 1.5) (layer B.Cu) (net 2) (status 80000))
 (segment (start 147.32 99.822) (end 146.939 99.441) (width 1.5) (layer B.Cu) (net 2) (status 80000))
 (segment (start 146.939 99.441) (end 147 99.5) (width 1.5) (layer B.Cu) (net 2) (status 80000))
 (segment (start 149.54 99.5) (end 149.479 99.441) (width 1.5) (layer B.Cu) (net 3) (status 80000))
 (segment (start 149.479 99.441) (end 149.479 95.377) (width 1.5) (layer B.Cu) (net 3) (status 80000))
 (segment (start 149.479 95.377) (end 146.939 92.837) (width 1.5) (layer B.Cu) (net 3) (status 80000))
 (segment (start 146.939 92.837) (end 147 92.9) (width 1.5) (layer B.Cu) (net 3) (status 80000))
 (segment (start 168.32 102.6) (end 168.275 102.616) (width 1.5) (layer B.Cu) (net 4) (status 80000))
 (segment (start 168.275 102.616) (end 168.275 102.362) (width 1.5) (layer B.Cu) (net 4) (status 80000))
 (segment (start 168.275 102.362) (end 152.273 86.36) (width 1.5) (layer B.Cu) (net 4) (status 80000))
 (segment (start 152.273 86.36) (end 143.256 86.36) (width 1.5) (layer B.Cu) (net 4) (status 80000))
 (segment (start 143.256 86.36) (end 143.129 86.487) (width 1.5) (layer B.Cu) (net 4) (status 80000))
 (segment (start 143.129 86.487) (end 142.113 86.487) (width 1.5) (layer B.Cu) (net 4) (status 80000))
 (segment (start 142.113 86.487) (end 140.589 88.011) (width 1.5) (layer B.Cu) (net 4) (status 80000))
 (segment (start 140.589 88.011) (end 140.589 89.027) (width 1.5) (layer B.Cu) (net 4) (status 80000))
 (segment (start 140.589 89.027) (end 140.462 89.154) (width 1.5) (layer B.Cu) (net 4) (status 80000))
 (segment (start 140.462 89.154) (end 140.462 108.839) (width 1.5) (layer B.Cu) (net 4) (status 80000))
 (segment (start 140.462 108.839) (end 144.399 112.776) (width 1.5) (layer B.Cu) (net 4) (status 80000))
 (segment (start 144.399 112.776) (end 156.972 112.776) (width 1.5) (layer B.Cu) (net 4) (status 80000))
 (segment (start 156.972 112.776) (end 157.099 112.649) (width 1.5) (layer B.Cu) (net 4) (status 80000))
 (segment (start 157.099 112.649) (end 158.115 112.649) (width 1.5) (layer B.Cu) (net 4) (status 80000))
 (segment (start 158.115 112.649) (end 160.528 110.236) (width 1.5) (layer B.Cu) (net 4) (status 80000))
 (segment (start 160.528 110.236) (end 160.655 110.236) (width 1.5) (layer B.Cu) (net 4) (status 80000))
 (segment (start 160.655 110.236) (end 160.7 110.22) (width 1.5) (layer B.Cu) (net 4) (status 80000))
 (segment (start 178.1 89.7) (end 178.054 89.662) (width 1.5) (layer B.Cu) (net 4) (status 80000))
 (segment (start 178.054 89.662) (end 178.054 98.806) (width 1.5) (layer B.Cu) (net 4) (status 80000))
 (segment (start 178.054 98.806) (end 173.482 103.378) (width 1.5) (layer B.Cu) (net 4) (status 80000))
 (segment (start 173.482 103.378) (end 173.5 103.4) (width 1.5) (layer B.Cu) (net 4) (status 80000))
 (segment (start 173.5 103.4) (end 173.482 103.378) (width 1.5) (layer B.Cu) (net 4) (status 80000))
 (segment (start 173.482 103.378) (end 172.72 102.616) (width 1.5) (layer B.Cu) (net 4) (status 80000))
 (segment (start 172.72 102.616) (end 168.275 102.616) (width 1.5) (layer B.Cu) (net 4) (status 80000))
 (segment (start 168.275 102.616) (end 168.32 102.6) (width 1.5) (layer B.Cu) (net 4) (status 80000))
 (segment (start 160.7 107.68) (end 160.655 107.696) (width 1.5) (layer B.Cu) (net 5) (status 80000))
 (segment (start 160.655 107.696) (end 160.274 108.077) (width 1.5) (layer B.Cu) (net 5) (status 80000))
 (segment (start 160.274 108.077) (end 158.623 108.077) (width 1.5) (layer B.Cu) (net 5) (status 80000))
 (segment (start 158.623 108.077) (end 156.083 110.617) (width 1.5) (layer B.Cu) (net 5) (status 80000))
 (segment (start 156.083 110.617) (end 146.304 110.617) (width 1.5) (layer B.Cu) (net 5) (status 80000))
 (segment (start 146.304 110.617) (end 146.304 109.093) (width 1.5) (layer B.Cu) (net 5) (status 80000))
 (segment (start 146.304 109.093) (end 144.399 107.188) (width 1.5) (layer B.Cu) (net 5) (status 80000))
 (segment (start 144.399 107.188) (end 144.399 105.664) (width 1.5) (layer B.Cu) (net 5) (status 80000))
 (segment (start 144.399 105.664) (end 143.51 104.775) (width 1.5) (layer B.Cu) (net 5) (status 80000))
 (segment (start 143.51 104.775) (end 143.51 104.648) (width 1.5) (layer B.Cu) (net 5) (status 80000))
 (segment (start 143.51 104.648) (end 143.383 104.521) (width 1.5) (layer B.Cu) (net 5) (status 80000))
 (segment (start 143.383 104.521) (end 143.383 104.394) (width 1.5) (layer B.Cu) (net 5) (status 80000))
 (segment (start 143.383 104.394) (end 142.748 103.759) (width 1.5) (layer B.Cu) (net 5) (status 80000))
 (segment (start 142.748 103.759) (end 142.748 102.743) (width 1.5) (layer B.Cu) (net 5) (status 80000))
 (segment (start 142.748 102.743) (end 142.621 102.616) (width 1.5) (layer B.Cu) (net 5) (status 80000))
 (segment (start 142.621 102.616) (end 142.621 90.043) (width 1.5) (layer B.Cu) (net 5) (status 80000))
 (segment (start 142.621 90.043) (end 144.145 88.519) (width 1.5) (layer B.Cu) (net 5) (status 80000))
 (segment (start 144.145 88.519) (end 148.717 88.519) (width 1.5) (layer B.Cu) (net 5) (status 80000))
 (segment (start 148.717 88.519) (end 148.844 88.646) (width 1.5) (layer B.Cu) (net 5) (status 80000))
 (segment (start 148.844 88.646) (end 149.86 88.646) (width 1.5) (layer B.Cu) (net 5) (status 80000))
 (segment (start 149.86 88.646) (end 152.527 91.313) (width 1.5) (layer B.Cu) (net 5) (status 80000))
 (segment (start 152.527 91.313) (end 152.654 91.313) (width 1.5) (layer B.Cu) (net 5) (status 80000))
 (segment (start 152.654 91.313) (end 154.178 92.837) (width 1.5) (layer B.Cu) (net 5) (status 80000))
 (segment (start 154.178 92.837) (end 154.559 92.837) (width 1.5) (layer B.Cu) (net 5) (status 80000))
 (segment (start 154.559 92.837) (end 154.62 92.9) (width 1.5) (layer B.Cu) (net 5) (status 80000))
 (segment (start 178.3 117.06) (end 178.308 117.094) (width 1.5) (layer B.Cu) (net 6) (status 80000))
 (segment (start 178.308 117.094) (end 178.689 116.713) (width 1.5) (layer B.Cu) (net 6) (status 80000))
 (segment (start 178.689 116.713) (end 180.467 116.713) (width 1.5) (layer B.Cu) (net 6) (status 80000))
 (segment (start 180.467 116.713) (end 180.467 108.077) (width 1.5) (layer B.Cu) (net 6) (status 80000))
 (segment (start 180.467 108.077) (end 180.975 107.569) (width 1.5) (layer B.Cu) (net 6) (status 80000))
 (segment (start 180.975 107.569) (end 180.975 106.553) (width 1.5) (layer B.Cu) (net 6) (status 80000))
 (segment (start 180.975 106.553) (end 181.864 105.664) (width 1.5) (layer B.Cu) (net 6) (status 80000))
 (segment (start 181.864 105.664) (end 181.864 104.14) (width 1.5) (layer B.Cu) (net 6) (status 80000))
 (segment (start 181.864 104.14) (end 181.102 103.378) (width 1.5) (layer B.Cu) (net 6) (status 80000))
 (segment (start 181.102 103.378) (end 181.12 103.4) (width 1.5) (layer B.Cu) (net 6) (status 80000))
 (segment (start 181.12 103.4) (end 181.102 103.378) (width 1.5) (layer B.Cu) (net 6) (status 80000))
 (segment (start 181.102 103.378) (end 178.943 105.537) (width 1.5) (layer B.Cu) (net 6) (status 80000))
 (segment (start 178.943 105.537) (end 172.466 105.537) (width 1.5) (layer B.Cu) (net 6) (status 80000))
 (segment (start 172.466 105.537) (end 172.085 105.156) (width 1.5) (layer B.Cu) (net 6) (status 80000))
 (segment (start 172.085 105.156) (end 168.275 105.156) (width 1.5) (layer B.Cu) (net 6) (status 80000))
 (segment (start 168.275 105.156) (end 168.32 105.14) (width 1.5) (layer B.Cu) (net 6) (status 80000))
 (segment (start 178.3 117.06) (end 178.308 117.094) (width 1.5) (layer B.Cu) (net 6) (status 80000))
 (segment (start 178.308 117.094) (end 178.308 119.634) (width 1.5) (layer B.Cu) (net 6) (status 80000))
 (segment (start 178.308 119.634) (end 178.3 119.6) (width 1.5) (layer B.Cu) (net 6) (status 80000)))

